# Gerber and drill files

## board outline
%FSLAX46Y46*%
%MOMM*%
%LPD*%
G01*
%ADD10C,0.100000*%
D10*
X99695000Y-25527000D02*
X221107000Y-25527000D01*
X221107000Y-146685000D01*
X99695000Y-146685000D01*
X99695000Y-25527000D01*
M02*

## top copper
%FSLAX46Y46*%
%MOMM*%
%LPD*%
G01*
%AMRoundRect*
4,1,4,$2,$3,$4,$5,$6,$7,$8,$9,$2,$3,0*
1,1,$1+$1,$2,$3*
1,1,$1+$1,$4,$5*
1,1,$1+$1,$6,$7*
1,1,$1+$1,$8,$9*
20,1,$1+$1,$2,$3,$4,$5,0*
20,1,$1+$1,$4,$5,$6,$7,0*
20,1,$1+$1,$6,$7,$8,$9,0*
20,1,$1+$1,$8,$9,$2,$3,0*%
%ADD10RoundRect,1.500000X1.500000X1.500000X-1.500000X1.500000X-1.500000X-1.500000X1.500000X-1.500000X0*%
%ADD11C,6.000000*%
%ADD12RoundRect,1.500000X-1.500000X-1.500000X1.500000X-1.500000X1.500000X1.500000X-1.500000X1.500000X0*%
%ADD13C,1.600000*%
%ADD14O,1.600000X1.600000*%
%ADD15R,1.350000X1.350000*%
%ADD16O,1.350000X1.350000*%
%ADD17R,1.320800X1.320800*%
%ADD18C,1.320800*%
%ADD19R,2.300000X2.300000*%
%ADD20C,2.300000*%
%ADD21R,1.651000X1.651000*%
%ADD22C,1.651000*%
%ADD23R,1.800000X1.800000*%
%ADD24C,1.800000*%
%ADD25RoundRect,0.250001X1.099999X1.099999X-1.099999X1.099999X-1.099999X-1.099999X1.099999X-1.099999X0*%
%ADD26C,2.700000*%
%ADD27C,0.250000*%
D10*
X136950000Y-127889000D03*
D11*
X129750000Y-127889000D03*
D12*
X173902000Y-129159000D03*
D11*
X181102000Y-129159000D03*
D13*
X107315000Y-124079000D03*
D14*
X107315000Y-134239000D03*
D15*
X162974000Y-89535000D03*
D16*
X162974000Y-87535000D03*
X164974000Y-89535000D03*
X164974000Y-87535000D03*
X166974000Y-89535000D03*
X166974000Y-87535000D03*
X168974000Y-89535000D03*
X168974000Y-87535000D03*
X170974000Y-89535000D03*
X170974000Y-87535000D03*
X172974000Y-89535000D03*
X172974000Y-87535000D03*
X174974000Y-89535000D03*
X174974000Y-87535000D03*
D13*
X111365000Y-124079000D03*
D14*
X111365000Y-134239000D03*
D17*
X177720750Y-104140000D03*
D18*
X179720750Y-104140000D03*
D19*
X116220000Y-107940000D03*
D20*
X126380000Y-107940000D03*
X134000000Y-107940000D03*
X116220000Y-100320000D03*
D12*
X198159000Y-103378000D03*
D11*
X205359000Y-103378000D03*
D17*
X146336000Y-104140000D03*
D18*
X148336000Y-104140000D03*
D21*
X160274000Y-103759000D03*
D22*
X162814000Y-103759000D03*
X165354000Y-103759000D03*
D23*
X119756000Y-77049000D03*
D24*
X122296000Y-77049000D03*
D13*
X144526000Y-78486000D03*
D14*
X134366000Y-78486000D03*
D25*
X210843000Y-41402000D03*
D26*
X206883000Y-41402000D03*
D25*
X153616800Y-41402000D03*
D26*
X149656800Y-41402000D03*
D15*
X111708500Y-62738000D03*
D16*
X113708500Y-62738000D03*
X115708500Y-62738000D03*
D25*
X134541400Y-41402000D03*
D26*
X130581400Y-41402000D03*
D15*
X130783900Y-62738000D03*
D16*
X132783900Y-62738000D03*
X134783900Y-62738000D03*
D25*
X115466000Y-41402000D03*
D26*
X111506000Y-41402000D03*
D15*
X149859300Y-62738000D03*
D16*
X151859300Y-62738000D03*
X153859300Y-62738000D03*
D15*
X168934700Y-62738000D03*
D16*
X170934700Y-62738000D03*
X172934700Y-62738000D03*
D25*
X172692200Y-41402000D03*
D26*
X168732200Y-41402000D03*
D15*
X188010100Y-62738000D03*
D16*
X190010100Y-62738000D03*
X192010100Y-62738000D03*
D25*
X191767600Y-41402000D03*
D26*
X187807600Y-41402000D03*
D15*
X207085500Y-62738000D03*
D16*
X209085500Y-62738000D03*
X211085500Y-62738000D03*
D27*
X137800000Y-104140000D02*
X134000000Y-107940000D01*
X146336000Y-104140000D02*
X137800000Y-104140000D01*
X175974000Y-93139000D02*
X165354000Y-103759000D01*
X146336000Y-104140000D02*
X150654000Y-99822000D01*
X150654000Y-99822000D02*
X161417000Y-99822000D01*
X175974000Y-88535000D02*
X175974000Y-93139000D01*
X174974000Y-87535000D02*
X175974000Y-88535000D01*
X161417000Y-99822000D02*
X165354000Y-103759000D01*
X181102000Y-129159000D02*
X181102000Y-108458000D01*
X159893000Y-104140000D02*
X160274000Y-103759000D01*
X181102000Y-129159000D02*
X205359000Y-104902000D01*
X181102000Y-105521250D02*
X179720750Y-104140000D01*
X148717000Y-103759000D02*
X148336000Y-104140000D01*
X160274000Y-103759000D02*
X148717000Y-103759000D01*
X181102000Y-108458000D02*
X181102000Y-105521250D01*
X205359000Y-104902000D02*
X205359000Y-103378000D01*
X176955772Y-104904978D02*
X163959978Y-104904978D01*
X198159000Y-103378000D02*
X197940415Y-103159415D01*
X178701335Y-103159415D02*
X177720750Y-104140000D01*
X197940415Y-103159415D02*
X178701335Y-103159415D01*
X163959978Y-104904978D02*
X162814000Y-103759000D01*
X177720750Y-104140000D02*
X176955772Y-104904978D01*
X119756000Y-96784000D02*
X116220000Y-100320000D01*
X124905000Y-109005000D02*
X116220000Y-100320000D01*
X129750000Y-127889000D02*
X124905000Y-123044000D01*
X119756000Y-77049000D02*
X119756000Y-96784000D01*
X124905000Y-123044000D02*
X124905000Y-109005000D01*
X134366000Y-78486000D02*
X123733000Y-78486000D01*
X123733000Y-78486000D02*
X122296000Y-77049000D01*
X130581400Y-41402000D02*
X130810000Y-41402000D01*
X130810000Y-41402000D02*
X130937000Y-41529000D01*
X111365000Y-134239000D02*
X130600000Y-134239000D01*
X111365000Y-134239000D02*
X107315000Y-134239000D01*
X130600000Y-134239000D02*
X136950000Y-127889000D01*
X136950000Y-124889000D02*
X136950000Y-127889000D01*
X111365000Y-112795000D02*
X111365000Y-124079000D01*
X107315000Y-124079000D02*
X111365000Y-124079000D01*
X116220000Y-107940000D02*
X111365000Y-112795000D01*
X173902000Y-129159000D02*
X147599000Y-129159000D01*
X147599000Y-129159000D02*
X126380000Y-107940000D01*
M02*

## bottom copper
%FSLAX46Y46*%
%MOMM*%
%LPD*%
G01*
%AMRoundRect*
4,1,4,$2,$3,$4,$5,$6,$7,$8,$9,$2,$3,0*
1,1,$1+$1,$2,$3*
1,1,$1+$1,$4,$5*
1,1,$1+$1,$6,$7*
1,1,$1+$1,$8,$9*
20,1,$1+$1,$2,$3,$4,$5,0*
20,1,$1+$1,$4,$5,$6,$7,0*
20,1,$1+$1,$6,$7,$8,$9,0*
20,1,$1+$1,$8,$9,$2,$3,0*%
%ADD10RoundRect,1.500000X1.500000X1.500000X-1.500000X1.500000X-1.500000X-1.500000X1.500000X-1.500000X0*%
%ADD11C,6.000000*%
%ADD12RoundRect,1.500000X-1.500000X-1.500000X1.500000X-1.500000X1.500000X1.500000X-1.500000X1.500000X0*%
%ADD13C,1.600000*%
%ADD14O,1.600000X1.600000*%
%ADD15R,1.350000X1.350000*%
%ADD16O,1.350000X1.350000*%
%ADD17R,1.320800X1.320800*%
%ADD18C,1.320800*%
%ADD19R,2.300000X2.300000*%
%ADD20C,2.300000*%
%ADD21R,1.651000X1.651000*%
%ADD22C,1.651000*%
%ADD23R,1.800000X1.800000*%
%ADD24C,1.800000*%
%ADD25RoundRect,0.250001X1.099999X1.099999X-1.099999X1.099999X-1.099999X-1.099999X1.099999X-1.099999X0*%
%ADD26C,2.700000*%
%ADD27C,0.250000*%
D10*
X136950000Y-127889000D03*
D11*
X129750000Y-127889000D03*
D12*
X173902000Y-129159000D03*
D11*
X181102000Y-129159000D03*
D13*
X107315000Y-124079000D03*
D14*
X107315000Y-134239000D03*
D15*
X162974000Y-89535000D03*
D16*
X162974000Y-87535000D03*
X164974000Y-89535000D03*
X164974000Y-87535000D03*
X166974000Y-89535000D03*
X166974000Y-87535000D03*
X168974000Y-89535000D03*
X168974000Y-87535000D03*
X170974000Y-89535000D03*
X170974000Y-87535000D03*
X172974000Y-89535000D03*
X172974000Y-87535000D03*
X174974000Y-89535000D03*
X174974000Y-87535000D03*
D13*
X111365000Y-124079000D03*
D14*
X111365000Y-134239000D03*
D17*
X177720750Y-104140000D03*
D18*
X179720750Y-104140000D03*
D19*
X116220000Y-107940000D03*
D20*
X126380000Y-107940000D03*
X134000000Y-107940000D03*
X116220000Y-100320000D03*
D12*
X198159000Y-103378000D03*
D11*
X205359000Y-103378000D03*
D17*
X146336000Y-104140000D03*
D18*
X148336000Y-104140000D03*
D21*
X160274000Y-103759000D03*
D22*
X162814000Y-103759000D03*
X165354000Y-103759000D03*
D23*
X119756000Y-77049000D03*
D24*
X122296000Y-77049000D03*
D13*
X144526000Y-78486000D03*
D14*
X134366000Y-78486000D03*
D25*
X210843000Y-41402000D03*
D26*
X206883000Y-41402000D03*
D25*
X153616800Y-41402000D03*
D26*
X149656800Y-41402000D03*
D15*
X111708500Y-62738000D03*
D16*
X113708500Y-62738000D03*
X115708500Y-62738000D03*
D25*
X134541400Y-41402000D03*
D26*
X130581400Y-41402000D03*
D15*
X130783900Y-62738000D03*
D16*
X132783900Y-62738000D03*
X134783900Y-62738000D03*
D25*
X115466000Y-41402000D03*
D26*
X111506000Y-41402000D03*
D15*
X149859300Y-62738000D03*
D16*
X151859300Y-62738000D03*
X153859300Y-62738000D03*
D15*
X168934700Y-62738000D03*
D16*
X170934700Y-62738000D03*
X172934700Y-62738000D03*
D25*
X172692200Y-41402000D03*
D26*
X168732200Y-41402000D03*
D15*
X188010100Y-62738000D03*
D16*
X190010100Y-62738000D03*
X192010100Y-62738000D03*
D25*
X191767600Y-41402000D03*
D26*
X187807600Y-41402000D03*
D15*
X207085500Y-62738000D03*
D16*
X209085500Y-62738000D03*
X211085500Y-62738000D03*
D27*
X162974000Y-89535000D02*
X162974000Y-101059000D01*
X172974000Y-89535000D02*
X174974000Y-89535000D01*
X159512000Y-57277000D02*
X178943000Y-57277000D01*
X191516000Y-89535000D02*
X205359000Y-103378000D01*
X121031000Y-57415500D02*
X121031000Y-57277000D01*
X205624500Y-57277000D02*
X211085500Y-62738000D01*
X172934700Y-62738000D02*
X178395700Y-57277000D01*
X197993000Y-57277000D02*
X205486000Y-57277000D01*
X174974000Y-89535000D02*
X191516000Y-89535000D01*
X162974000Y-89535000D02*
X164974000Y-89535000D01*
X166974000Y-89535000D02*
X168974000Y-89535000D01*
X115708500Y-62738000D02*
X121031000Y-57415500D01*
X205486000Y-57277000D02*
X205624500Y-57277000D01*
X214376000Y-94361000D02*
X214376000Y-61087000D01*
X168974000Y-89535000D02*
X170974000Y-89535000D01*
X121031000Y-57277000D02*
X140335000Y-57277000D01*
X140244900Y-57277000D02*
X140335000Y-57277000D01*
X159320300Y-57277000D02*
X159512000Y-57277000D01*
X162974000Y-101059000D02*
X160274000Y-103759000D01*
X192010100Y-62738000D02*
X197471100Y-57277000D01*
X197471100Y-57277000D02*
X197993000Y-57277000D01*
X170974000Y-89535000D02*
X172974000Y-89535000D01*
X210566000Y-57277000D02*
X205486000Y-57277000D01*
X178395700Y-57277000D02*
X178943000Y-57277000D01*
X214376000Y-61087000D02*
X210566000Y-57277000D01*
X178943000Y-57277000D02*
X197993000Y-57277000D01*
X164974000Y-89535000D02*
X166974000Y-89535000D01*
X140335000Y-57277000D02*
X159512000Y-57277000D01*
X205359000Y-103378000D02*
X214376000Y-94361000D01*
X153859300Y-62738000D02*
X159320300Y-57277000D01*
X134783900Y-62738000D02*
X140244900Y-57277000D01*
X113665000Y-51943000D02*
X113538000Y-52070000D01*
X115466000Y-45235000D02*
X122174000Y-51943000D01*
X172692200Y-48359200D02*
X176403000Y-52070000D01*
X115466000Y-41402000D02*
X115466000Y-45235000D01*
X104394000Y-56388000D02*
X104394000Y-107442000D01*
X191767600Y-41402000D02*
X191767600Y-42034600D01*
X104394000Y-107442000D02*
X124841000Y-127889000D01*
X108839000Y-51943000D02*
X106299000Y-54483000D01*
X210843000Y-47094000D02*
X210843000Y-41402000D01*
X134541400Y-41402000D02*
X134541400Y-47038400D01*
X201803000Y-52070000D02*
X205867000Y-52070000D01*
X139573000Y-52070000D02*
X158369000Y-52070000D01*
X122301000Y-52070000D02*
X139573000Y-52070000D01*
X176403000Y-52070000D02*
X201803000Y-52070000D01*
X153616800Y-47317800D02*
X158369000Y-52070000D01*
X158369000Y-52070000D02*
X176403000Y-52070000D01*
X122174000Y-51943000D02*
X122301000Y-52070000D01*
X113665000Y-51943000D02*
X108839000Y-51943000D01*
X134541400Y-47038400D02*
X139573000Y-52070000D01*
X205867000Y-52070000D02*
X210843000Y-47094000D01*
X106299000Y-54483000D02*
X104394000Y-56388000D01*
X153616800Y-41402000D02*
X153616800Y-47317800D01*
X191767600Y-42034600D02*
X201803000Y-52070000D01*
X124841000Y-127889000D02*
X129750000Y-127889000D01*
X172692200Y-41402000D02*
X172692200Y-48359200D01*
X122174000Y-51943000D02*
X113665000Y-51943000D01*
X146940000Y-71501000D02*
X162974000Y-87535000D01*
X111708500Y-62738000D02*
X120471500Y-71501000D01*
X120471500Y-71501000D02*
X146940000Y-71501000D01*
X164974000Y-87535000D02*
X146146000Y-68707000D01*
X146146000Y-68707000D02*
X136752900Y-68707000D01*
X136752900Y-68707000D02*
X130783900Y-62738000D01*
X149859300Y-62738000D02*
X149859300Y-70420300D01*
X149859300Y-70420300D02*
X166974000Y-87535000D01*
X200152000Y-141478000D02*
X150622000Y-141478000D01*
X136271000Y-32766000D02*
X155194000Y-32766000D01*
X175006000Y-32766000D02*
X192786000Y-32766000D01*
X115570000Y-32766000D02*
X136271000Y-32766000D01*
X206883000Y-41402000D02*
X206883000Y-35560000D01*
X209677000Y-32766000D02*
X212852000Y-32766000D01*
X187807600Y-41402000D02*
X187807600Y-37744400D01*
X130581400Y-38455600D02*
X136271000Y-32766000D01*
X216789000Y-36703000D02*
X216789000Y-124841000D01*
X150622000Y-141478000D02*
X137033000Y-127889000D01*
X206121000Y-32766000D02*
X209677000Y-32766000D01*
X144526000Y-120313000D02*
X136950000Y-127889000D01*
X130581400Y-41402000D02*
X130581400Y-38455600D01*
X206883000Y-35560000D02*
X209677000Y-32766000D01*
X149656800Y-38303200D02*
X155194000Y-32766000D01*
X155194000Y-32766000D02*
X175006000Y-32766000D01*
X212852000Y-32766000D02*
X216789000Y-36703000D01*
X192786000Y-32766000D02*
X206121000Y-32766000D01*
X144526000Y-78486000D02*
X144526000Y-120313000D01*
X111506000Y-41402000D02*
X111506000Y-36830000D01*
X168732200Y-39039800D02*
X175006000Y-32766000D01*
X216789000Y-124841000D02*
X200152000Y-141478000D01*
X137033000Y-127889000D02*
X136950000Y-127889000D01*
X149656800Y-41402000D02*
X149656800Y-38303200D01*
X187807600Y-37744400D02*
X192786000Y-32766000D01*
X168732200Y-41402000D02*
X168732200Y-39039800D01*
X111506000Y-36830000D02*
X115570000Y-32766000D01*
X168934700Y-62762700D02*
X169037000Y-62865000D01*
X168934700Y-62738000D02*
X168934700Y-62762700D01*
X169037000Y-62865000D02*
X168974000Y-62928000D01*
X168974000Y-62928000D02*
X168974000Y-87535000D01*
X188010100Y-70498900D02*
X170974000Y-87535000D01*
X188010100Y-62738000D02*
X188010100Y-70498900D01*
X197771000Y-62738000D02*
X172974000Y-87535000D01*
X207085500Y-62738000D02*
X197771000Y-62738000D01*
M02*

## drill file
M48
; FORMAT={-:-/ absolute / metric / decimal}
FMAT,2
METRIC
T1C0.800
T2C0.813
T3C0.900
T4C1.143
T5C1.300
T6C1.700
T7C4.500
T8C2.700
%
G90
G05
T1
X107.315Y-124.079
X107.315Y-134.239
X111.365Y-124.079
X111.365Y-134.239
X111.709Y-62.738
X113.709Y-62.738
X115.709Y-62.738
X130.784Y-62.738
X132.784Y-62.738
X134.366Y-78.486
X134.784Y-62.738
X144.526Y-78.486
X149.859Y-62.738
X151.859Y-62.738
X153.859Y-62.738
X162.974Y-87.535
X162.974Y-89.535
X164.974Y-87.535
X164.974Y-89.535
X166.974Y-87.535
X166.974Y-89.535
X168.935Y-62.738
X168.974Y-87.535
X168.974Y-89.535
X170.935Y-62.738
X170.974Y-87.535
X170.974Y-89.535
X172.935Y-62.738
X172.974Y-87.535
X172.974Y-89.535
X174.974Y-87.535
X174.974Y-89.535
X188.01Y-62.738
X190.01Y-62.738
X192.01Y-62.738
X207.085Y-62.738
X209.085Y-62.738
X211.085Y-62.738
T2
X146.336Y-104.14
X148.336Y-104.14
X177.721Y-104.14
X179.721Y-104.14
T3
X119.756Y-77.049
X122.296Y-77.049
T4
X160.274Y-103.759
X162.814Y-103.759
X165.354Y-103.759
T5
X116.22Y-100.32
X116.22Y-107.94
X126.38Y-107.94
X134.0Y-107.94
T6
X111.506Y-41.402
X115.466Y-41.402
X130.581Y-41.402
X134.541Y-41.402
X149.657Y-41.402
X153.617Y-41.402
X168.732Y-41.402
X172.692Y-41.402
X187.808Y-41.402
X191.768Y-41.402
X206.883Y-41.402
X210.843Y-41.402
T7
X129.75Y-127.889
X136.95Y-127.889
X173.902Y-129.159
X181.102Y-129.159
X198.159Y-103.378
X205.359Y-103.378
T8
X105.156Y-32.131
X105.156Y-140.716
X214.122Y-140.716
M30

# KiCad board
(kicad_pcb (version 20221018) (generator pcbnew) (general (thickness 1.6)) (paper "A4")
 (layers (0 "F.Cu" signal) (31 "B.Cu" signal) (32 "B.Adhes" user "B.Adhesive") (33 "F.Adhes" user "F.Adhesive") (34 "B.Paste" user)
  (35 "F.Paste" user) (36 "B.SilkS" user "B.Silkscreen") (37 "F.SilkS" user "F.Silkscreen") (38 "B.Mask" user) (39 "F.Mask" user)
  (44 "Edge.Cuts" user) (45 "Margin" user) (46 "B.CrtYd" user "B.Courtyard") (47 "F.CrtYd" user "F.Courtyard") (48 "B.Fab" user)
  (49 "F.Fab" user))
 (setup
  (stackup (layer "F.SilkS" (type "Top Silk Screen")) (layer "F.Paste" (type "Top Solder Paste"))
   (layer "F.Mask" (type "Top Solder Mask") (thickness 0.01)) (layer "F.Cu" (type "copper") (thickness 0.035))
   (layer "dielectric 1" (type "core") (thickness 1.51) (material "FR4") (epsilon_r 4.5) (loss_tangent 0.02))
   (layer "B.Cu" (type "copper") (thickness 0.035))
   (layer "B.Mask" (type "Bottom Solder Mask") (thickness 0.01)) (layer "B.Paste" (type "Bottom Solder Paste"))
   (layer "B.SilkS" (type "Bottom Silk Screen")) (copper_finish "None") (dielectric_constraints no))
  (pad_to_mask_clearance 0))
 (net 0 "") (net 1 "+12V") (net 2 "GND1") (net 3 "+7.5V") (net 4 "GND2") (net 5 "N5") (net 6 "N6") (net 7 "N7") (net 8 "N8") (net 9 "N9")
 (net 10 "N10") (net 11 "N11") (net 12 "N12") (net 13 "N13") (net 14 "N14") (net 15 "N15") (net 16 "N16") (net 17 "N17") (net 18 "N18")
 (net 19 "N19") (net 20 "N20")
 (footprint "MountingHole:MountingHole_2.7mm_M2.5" (layer "F.Cu") (at 214.122 140.716)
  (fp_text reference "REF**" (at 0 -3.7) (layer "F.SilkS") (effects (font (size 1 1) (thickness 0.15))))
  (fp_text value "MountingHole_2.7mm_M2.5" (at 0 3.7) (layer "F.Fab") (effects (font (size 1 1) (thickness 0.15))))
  (pad "" np_thru_hole circle (at 0 0) (size 2.7 2.7) (drill 2.7) (layers "F&B.Cu" "*.Mask")))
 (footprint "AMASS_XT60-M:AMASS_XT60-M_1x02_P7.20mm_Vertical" (layer "F.Cu") (at 136.95 127.889 180)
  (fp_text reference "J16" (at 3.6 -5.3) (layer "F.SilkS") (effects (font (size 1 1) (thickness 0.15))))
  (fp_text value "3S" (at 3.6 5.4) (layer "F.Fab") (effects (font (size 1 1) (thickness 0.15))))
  (pad "1" thru_hole roundrect (at 0 0 180) (size 6 6) (drill 4.5) (layers "*.Cu" "*.Mask") (roundrect_rratio 0.25) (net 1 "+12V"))
  (pad "2" thru_hole circle (at 7.2 0 180) (size 6 6) (drill 4.5) (layers "*.Cu" "*.Mask") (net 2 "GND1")))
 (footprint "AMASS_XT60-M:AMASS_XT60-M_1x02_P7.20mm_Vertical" (layer "F.Cu") (at 173.902 129.159)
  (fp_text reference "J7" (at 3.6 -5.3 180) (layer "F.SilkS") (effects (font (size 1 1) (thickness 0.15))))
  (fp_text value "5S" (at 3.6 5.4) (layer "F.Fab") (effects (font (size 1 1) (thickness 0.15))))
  (pad "1" thru_hole roundrect (at 0 0) (size 6 6) (drill 4.5) (layers "*.Cu" "*.Mask") (roundrect_rratio 0.25) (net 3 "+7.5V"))
  (pad "2" thru_hole circle (at 7.2 0) (size 6 6) (drill 4.5) (layers "*.Cu" "*.Mask") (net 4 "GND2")))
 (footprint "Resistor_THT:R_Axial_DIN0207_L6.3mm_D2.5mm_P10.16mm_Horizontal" (layer "F.Cu") (at 107.315 124.079 -90)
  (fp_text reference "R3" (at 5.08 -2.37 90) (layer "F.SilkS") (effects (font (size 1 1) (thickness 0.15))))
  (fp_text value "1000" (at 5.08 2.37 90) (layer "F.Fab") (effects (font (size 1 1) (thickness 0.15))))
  (pad "1" thru_hole circle (at 0 0 270) (size 1.6 1.6) (drill 0.8) (layers "*.Cu" "*.Mask") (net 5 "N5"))
  (pad "2" thru_hole oval (at 10.16 0 270) (size 1.6 1.6) (drill 0.8) (layers "*.Cu" "*.Mask") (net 1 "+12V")))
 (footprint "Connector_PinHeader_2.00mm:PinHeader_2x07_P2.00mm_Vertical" (layer "F.Cu") (at 162.974 89.535 90)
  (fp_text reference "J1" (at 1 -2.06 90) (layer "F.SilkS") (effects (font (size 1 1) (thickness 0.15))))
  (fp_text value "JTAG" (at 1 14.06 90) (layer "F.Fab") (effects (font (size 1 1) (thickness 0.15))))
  (pad "1" thru_hole rect (at 0 0 90) (size 1.35 1.35) (drill 0.8) (layers "*.Cu" "*.Mask") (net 4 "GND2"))
  (pad "2" thru_hole oval (at 2 0 90) (size 1.35 1.35) (drill 0.8) (layers "*.Cu" "*.Mask") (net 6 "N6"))
  (pad "3" thru_hole oval (at 0 2 90) (size 1.35 1.35) (drill 0.8) (layers "*.Cu" "*.Mask") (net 4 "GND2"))
  (pad "4" thru_hole oval (at 2 2 90) (size 1.35 1.35) (drill 0.8) (layers "*.Cu" "*.Mask") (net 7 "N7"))
  (pad "5" thru_hole oval (at 0 4 90) (size 1.35 1.35) (drill 0.8) (layers "*.Cu" "*.Mask") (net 4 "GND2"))
  (pad "6" thru_hole oval (at 2 4 90) (size 1.35 1.35) (drill 0.8) (layers "*.Cu" "*.Mask") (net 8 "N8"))
  (pad "7" thru_hole oval (at 0 6 90) (size 1.35 1.35) (drill 0.8) (layers "*.Cu" "*.Mask") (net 4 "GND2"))
  (pad "8" thru_hole oval (at 2 6 90) (size 1.35 1.35) (drill 0.8) (layers "*.Cu" "*.Mask") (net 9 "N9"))
  (pad "9" thru_hole oval (at 0 8 90) (size 1.35 1.35) (drill 0.8) (layers "*.Cu" "*.Mask") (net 4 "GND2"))
  (pad "10" thru_hole oval (at 2 8 90) (size 1.35 1.35) (drill 0.8) (layers "*.Cu" "*.Mask") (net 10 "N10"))
  (pad "11" thru_hole oval (at 0 10 90) (size 1.35 1.35) (drill 0.8) (layers "*.Cu" "*.Mask") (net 4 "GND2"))
  (pad "12" thru_hole oval (at 2 10 90) (size 1.35 1.35) (drill 0.8) (layers "*.Cu" "*.Mask") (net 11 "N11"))
  (pad "13" thru_hole oval (at 0 12 90) (size 1.35 1.35) (drill 0.8) (layers "*.Cu" "*.Mask") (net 4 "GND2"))
  (pad "14" thru_hole oval (at 2 12 90) (size 1.35 1.35) (drill 0.8) (layers "*.Cu" "*.Mask") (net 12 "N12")))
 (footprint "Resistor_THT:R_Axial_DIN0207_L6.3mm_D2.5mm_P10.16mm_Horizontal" (layer "F.Cu") (at 111.365 124.079 -90)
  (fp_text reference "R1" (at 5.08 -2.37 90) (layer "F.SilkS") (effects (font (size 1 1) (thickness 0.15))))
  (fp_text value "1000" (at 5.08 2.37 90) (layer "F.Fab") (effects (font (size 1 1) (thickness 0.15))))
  (pad "1" thru_hole circle (at 0 0 270) (size 1.6 1.6) (drill 0.8) (layers "*.Cu" "*.Mask") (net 5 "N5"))
  (pad "2" thru_hole oval (at 10.16 0 270) (size 1.6 1.6) (drill 0.8) (layers "*.Cu" "*.Mask") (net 1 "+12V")))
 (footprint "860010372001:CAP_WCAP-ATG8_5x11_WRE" (layer "F.Cu") (at 177.72075 104.14)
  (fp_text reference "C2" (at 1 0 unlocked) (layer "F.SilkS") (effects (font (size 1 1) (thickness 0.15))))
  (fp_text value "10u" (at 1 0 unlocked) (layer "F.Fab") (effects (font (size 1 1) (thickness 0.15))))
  (pad "1" thru_hole rect (at 0 0) (size 1.3208 1.3208) (drill 0.8128) (layers "*.Cu" "*.Mask") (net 12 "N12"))
  (pad "2" thru_hole circle (at 2 0) (size 1.3208 1.3208) (drill 0.8128) (layers "*.Cu" "*.Mask") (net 4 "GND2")))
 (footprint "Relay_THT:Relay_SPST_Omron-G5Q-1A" (layer "F.Cu") (at 116.22 107.94)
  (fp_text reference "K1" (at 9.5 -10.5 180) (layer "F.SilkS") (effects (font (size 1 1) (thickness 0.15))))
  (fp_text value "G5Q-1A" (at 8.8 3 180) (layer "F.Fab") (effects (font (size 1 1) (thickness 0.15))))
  (pad "1" thru_hole rect (at 0 0 180) (size 2.3 2.3) (drill 1.3) (layers "*.Cu" "*.Mask") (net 5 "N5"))
  (pad "2" thru_hole circle (at 10.16 0 180) (size 2.3 2.3) (drill 1.3) (layers "*.Cu" "*.Mask") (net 3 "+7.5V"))
  (pad "3" thru_hole circle (at 17.78 0 180) (size 2.3 2.3) (drill 1.3) (layers "*.Cu" "*.Mask") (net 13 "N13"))
  (pad "5" thru_hole circle (at 0 -7.62 180) (size 2.3 2.3) (drill 1.3) (layers "*.Cu" "*.Mask") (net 2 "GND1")))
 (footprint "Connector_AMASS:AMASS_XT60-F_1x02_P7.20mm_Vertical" (layer "F.Cu") (at 198.159 103.378)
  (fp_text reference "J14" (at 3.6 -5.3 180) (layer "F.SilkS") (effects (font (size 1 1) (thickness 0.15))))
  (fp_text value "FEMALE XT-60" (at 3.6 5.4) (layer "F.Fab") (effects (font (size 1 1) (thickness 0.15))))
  (pad "1" thru_hole roundrect (at 0 0) (size 6 6) (drill 4.5) (layers "*.Cu" "*.Mask") (roundrect_rratio 0.25) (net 12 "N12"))
  (pad "2" thru_hole circle (at 7.2 0) (size 6 6) (drill 4.5) (layers "*.Cu" "*.Mask") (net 4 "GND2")))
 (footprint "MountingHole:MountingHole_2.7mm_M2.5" (layer "F.Cu") (at 105.156 140.716)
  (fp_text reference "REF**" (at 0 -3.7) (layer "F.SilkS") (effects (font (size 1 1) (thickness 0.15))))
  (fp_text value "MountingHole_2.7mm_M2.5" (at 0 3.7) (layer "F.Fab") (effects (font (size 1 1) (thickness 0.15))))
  (pad "" np_thru_hole circle (at 0 0) (size 2.7 2.7) (drill 2.7) (layers "F&B.Cu" "*.Mask")))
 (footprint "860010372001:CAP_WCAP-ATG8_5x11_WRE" (layer "F.Cu") (at 146.336 104.14)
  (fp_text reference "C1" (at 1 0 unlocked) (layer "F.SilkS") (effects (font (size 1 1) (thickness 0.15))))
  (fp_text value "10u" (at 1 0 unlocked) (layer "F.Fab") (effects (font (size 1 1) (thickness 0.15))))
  (pad "1" thru_hole rect (at 0 0) (size 1.3208 1.3208) (drill 0.8128) (layers "*.Cu" "*.Mask") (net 13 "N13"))
  (pad "2" thru_hole circle (at 2 0) (size 1.3208 1.3208) (drill 0.8128) (layers "*.Cu" "*.Mask") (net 4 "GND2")))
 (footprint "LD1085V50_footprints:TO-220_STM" (layer "F.Cu") (at 160.274 103.759)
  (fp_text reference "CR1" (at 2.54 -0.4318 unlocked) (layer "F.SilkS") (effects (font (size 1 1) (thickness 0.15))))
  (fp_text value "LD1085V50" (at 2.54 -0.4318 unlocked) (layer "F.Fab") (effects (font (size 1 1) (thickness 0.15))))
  (pad "1" thru_hole rect (at 0 0) (size 1.651 1.651) (drill 1.143) (layers "*.Cu" "*.Mask") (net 4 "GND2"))
  (pad "2" thru_hole circle (at 2.54 0) (size 1.651 1.651) (drill 1.143) (layers "*.Cu" "*.Mask") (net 12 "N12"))
  (pad "3" thru_hole circle (at 5.08 0) (size 1.651 1.651) (drill 1.143) (layers "*.Cu" "*.Mask") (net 13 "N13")))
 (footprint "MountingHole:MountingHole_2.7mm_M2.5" (layer "F.Cu") (at 105.156 32.131)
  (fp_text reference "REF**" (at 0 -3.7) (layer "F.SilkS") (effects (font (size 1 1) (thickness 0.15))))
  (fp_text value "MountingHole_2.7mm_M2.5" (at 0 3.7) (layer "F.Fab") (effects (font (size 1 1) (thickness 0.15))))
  (pad "" np_thru_hole circle (at 0 0) (size 2.7 2.7) (drill 2.7) (layers "*.Cu" "*.Mask")))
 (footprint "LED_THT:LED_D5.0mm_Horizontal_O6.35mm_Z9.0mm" (layer "F.Cu") (at 119.756 77.049)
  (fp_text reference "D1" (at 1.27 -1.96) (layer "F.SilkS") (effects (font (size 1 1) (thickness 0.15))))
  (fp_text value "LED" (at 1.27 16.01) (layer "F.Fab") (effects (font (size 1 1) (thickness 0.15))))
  (pad "1" thru_hole rect (at 0 0) (size 1.8 1.8) (drill 0.9) (layers "*.Cu" "*.Mask") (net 2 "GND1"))
  (pad "2" thru_hole circle (at 2.54 0) (size 1.8 1.8) (drill 0.9) (layers "*.Cu" "*.Mask") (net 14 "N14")))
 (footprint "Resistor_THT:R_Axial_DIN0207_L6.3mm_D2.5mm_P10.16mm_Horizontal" (layer "F.Cu") (at 144.526 78.486 180)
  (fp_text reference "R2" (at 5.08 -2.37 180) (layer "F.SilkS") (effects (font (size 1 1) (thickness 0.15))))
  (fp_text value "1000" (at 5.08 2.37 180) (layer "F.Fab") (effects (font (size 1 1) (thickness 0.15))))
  (pad "1" thru_hole circle (at 0 0 180) (size 1.6 1.6) (drill 0.8) (layers "*.Cu" "*.Mask") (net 1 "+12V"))
  (pad "2" thru_hole oval (at 10.16 0 180) (size 1.6 1.6) (drill 0.8) (layers "*.Cu" "*.Mask") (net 14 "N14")))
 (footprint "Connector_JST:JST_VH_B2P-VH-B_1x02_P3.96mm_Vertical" (layer "B.Cu") (at 210.843 41.402 180)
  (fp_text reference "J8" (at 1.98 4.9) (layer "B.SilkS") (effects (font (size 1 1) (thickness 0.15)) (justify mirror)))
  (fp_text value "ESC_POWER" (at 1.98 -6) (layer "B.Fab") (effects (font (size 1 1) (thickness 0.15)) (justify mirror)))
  (pad "1" thru_hole roundrect (at 0 0 180) (size 2.7 2.7) (drill 1.7) (layers "*.Cu" "*.Mask") (roundrect_rratio 0.09259296296)
   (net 2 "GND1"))
  (pad "2" thru_hole circle (at 3.96 0 180) (size 2.7 2.7) (drill 1.7) (layers "*.Cu" "*.Mask") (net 1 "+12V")))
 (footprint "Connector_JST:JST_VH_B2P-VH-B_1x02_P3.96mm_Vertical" (layer "B.Cu") (at 153.6168 41.402 180)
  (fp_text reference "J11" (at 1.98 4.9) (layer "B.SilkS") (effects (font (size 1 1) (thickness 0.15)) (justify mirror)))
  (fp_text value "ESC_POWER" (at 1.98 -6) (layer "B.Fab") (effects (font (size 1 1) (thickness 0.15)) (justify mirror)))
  (pad "1" thru_hole roundrect (at 0 0 180) (size 2.7 2.7) (drill 1.7) (layers "*.Cu" "*.Mask") (roundrect_rratio 0.09259296296)
   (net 2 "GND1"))
  (pad "2" thru_hole circle (at 3.96 0 180) (size 2.7 2.7) (drill 1.7) (layers "*.Cu" "*.Mask") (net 1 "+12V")))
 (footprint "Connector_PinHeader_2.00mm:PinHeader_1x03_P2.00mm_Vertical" (layer "B.Cu") (at 111.7085 62.738 -90)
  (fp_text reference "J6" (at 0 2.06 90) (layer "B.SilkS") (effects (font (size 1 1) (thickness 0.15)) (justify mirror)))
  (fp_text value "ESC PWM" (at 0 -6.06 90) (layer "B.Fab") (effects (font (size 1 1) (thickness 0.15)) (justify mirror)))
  (pad "1" thru_hole rect (at 0 0 270) (size 1.35 1.35) (drill 0.8) (layers "*.Cu" "*.Mask") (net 6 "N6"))
  (pad "2" thru_hole oval (at 0 -2 270) (size 1.35 1.35) (drill 0.8) (layers "*.Cu" "*.Mask") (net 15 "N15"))
  (pad "3" thru_hole oval (at 0 -4 270) (size 1.35 1.35) (drill 0.8) (layers "*.Cu" "*.Mask") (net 4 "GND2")))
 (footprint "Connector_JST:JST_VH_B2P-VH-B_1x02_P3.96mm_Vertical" (layer "B.Cu") (at 134.5414 41.402 180)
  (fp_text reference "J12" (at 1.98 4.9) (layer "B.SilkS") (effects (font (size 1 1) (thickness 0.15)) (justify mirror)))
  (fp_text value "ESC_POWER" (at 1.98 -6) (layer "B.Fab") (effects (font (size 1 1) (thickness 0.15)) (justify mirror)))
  (pad "1" thru_hole roundrect (at 0 0 180) (size 2.7 2.7) (drill 1.7) (layers "*.Cu" "*.Mask") (roundrect_rratio 0.09259296296)
   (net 2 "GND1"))
  (pad "2" thru_hole circle (at 3.96 0 180) (size 2.7 2.7) (drill 1.7) (layers "*.Cu" "*.Mask") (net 1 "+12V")))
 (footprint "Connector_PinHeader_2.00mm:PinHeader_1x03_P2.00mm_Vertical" (layer "B.Cu") (at 130.7839 62.738 -90)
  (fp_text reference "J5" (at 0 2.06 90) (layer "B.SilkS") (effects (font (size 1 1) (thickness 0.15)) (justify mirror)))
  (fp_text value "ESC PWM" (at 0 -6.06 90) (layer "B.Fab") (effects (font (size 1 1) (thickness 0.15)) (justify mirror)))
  (pad "1" thru_hole rect (at 0 0 270) (size 1.35 1.35) (drill 0.8) (layers "*.Cu" "*.Mask") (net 7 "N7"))
  (pad "2" thru_hole oval (at 0 -2 270) (size 1.35 1.35) (drill 0.8) (layers "*.Cu" "*.Mask") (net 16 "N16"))
  (pad "3" thru_hole oval (at 0 -4 270) (size 1.35 1.35) (drill 0.8) (layers "*.Cu" "*.Mask") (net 4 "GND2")))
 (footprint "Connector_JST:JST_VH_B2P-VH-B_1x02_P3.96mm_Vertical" (layer "B.Cu") (at 115.466 41.402 180)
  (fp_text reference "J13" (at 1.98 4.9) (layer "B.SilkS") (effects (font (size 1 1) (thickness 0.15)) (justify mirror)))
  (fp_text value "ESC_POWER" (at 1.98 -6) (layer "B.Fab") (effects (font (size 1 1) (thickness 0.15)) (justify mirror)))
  (pad "1" thru_hole roundrect (at 0 0 180) (size 2.7 2.7) (drill 1.7) (layers "*.Cu" "*.Mask") (roundrect_rratio 0.09259296296)
   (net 2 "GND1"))
  (pad "2" thru_hole circle (at 3.96 0 180) (size 2.7 2.7) (drill 1.7) (layers "*.Cu" "*.Mask") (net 1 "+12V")))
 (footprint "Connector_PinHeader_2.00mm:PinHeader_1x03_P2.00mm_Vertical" (layer "B.Cu") (at 149.8593 62.738 -90)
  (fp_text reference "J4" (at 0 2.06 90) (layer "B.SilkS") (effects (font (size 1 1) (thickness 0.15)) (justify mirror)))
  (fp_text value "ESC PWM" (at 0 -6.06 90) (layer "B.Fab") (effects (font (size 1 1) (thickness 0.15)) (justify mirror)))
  (pad "1" thru_hole rect (at 0 0 270) (size 1.35 1.35) (drill 0.8) (layers "*.Cu" "*.Mask") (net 8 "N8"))
  (pad "2" thru_hole oval (at 0 -2 270) (size 1.35 1.35) (drill 0.8) (layers "*.Cu" "*.Mask") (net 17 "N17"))
  (pad "3" thru_hole oval (at 0 -4 270) (size 1.35 1.35) (drill 0.8) (layers "*.Cu" "*.Mask") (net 4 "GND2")))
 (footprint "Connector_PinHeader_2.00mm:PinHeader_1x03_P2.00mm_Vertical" (layer "B.Cu") (at 168.9347 62.738 -90)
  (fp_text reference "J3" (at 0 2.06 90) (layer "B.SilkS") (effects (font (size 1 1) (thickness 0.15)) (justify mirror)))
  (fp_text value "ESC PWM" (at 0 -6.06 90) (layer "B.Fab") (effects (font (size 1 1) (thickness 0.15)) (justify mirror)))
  (pad "1" thru_hole rect (at 0 0 270) (size 1.35 1.35) (drill 0.8) (layers "*.Cu" "*.Mask") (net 9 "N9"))
  (pad "2" thru_hole oval (at 0 -2 270) (size 1.35 1.35) (drill 0.8) (layers "*.Cu" "*.Mask") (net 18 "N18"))
  (pad "3" thru_hole oval (at 0 -4 270) (size 1.35 1.35) (drill 0.8) (layers "*.Cu" "*.Mask") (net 4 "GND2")))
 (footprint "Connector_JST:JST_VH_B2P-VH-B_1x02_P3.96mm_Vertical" (layer "B.Cu") (at 172.6922 41.402 180)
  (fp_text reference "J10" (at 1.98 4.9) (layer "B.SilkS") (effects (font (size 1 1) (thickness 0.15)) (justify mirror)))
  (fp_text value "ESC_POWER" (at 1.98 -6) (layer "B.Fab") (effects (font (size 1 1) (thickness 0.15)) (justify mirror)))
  (pad "1" thru_hole roundrect (at 0 0 180) (size 2.7 2.7) (drill 1.7) (layers "*.Cu" "*.Mask") (roundrect_rratio 0.09259296296)
   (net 2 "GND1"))
  (pad "2" thru_hole circle (at 3.96 0 180) (size 2.7 2.7) (drill 1.7) (layers "*.Cu" "*.Mask") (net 1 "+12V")))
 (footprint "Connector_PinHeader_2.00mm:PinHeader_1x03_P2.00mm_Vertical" (layer "B.Cu") (at 188.0101 62.738 -90)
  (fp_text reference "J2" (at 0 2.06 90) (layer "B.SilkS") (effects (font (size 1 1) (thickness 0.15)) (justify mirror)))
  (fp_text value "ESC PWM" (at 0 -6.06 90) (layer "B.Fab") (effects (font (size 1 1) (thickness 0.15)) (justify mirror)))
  (pad "1" thru_hole rect (at 0 0 270) (size 1.35 1.35) (drill 0.8) (layers "*.Cu" "*.Mask") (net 10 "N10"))
  (pad "2" thru_hole oval (at 0 -2 270) (size 1.35 1.35) (drill 0.8) (layers "*.Cu" "*.Mask") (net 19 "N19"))
  (pad "3" thru_hole oval (at 0 -4 270) (size 1.35 1.35) (drill 0.8) (layers "*.Cu" "*.Mask") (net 4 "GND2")))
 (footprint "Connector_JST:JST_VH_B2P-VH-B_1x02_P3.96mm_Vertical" (layer "B.Cu") (at 191.7676 41.402 180)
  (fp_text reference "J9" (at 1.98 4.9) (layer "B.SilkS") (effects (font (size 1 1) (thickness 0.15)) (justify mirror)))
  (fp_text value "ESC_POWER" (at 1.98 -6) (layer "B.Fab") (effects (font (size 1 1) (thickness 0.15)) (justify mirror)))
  (pad "1" thru_hole roundrect (at 0 0 180) (size 2.7 2.7) (drill 1.7) (layers "*.Cu" "*.Mask") (roundrect_rratio 0.09259296296)
   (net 2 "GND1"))
  (pad "2" thru_hole circle (at 3.96 0 180) (size 2.7 2.7) (drill 1.7) (layers "*.Cu" "*.Mask") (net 1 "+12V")))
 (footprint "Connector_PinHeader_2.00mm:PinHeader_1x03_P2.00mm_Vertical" (layer "B.Cu") (at 207.0855 62.738 -90)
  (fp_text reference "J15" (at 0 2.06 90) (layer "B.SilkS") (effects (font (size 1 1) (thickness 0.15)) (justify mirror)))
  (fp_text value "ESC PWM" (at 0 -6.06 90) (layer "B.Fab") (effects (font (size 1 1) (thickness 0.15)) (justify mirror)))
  (pad "1" thru_hole rect (at 0 0 270) (size 1.35 1.35) (drill 0.8) (layers "*.Cu" "*.Mask") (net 11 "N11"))
  (pad "2" thru_hole oval (at 0 -2 270) (size 1.35 1.35) (drill 0.8) (layers "*.Cu" "*.Mask") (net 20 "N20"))
  (pad "3" thru_hole oval (at 0 -4 270) (size 1.35 1.35) (drill 0.8) (layers "*.Cu" "*.Mask") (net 4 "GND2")))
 (gr_rect (start 99.695 25.527) (end 221.107 146.685) (stroke (width 0.1) (type default)) (fill none) (layer "Edge.Cuts"))
 (segment (start 137.8 104.14) (end 134 107.94) (width 0.25) (layer "F.Cu") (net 13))
 (segment (start 146.336 104.14) (end 137.8 104.14) (width 0.25) (layer "F.Cu") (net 13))
 (segment (start 175.974 93.139) (end 165.354 103.759) (width 0.25) (layer "F.Cu") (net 13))
 (segment (start 146.336 104.14) (end 150.654 99.822) (width 0.25) (layer "F.Cu") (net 13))
 (segment (start 150.654 99.822) (end 161.417 99.822) (width 0.25) (layer "F.Cu") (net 13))
 (segment (start 175.974 88.535) (end 175.974 93.139) (width 0.25) (layer "F.Cu") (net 13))
 (segment (start 174.974 87.535) (end 175.974 88.535) (width 0.25) (layer "F.Cu") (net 13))
 (segment (start 161.417 99.822) (end 165.354 103.759) (width 0.25) (layer "F.Cu") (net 13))
 (segment (start 181.102 129.159) (end 181.102 108.458) (width 0.25) (layer "F.Cu") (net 4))
 (segment (start 159.893 104.14) (end 160.274 103.759) (width 0.25) (layer "F.Cu") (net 4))
 (segment (start 181.102 129.159) (end 205.359 104.902) (width 0.25) (layer "F.Cu") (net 4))
 (segment (start 181.102 105.52125) (end 179.72075 104.14) (width 0.25) (layer "F.Cu") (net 4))
 (segment (start 148.717 103.759) (end 148.336 104.14) (width 0.25) (layer "F.Cu") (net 4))
 (segment (start 160.274 103.759) (end 148.717 103.759) (width 0.25) (layer "F.Cu") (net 4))
 (segment (start 181.102 108.458) (end 181.102 105.52125) (width 0.25) (layer "F.Cu") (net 4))
 (segment (start 205.359 104.902) (end 205.359 103.378) (width 0.25) (layer "F.Cu") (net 4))
 (segment (start 162.974 89.535) (end 162.974 101.059) (width 0.25) (layer "B.Cu") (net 4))
 (segment (start 172.974 89.535) (end 174.974 89.535) (width 0.25) (layer "B.Cu") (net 4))
 (segment (start 159.512 57.277) (end 178.943 57.277) (width 0.25) (layer "B.Cu") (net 4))
 (segment (start 191.516 89.535) (end 205.359 103.378) (width 0.25) (layer "B.Cu") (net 4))
 (segment (start 121.031 57.4155) (end 121.031 57.277) (width 0.25) (layer "B.Cu") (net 4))
 (segment (start 205.6245 57.277) (end 211.0855 62.738) (width 0.25) (layer "B.Cu") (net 4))
 (segment (start 172.9347 62.738) (end 178.3957 57.277) (width 0.25) (layer "B.Cu") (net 4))
 (segment (start 197.993 57.277) (end 205.486 57.277) (width 0.25) (layer "B.Cu") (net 4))
 (segment (start 174.974 89.535) (end 191.516 89.535) (width 0.25) (layer "B.Cu") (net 4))
 (segment (start 162.974 89.535) (end 164.974 89.535) (width 0.25) (layer "B.Cu") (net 4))
 (segment (start 166.974 89.535) (end 168.974 89.535) (width 0.25) (layer "B.Cu") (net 4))
 (segment (start 115.7085 62.738) (end 121.031 57.4155) (width 0.25) (layer "B.Cu") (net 4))
 (segment (start 205.486 57.277) (end 205.6245 57.277) (width 0.25) (layer "B.Cu") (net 4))
 (segment (start 214.376 94.361) (end 214.376 61.087) (width 0.25) (layer "B.Cu") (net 4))
 (segment (start 168.974 89.535) (end 170.974 89.535) (width 0.25) (layer "B.Cu") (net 4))
 (segment (start 121.031 57.277) (end 140.335 57.277) (width 0.25) (layer "B.Cu") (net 4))
 (segment (start 140.2449 57.277) (end 140.335 57.277) (width 0.25) (layer "B.Cu") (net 4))
 (segment (start 159.3203 57.277) (end 159.512 57.277) (width 0.25) (layer "B.Cu") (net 4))
 (segment (start 162.974 101.059) (end 160.274 103.759) (width 0.25) (layer "B.Cu") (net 4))
 (segment (start 192.0101 62.738) (end 197.4711 57.277) (width 0.25) (layer "B.Cu") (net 4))
 (segment (start 197.4711 57.277) (end 197.993 57.277) (width 0.25) (layer "B.Cu") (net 4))
 (segment (start 170.974 89.535) (end 172.974 89.535) (width 0.25) (layer "B.Cu") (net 4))
 (segment (start 210.566 57.277) (end 205.486 57.277) (width 0.25) (layer "B.Cu") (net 4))
 (segment (start 178.3957 57.277) (end 178.943 57.277) (width 0.25) (layer "B.Cu") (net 4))
 (segment (start 214.376 61.087) (end 210.566 57.277) (width 0.25) (layer "B.Cu") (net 4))
 (segment (start 178.943 57.277) (end 197.993 57.277) (width 0.25) (layer "B.Cu") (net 4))
 (segment (start 164.974 89.535) (end 166.974 89.535) (width 0.25) (layer "B.Cu") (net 4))
 (segment (start 140.335 57.277) (end 159.512 57.277) (width 0.25) (layer "B.Cu") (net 4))
 (segment (start 205.359 103.378) (end 214.376 94.361) (width 0.25) (layer "B.Cu") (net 4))
 (segment (start 153.8593 62.738) (end 159.3203 57.277) (width 0.25) (layer "B.Cu") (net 4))
 (segment (start 134.7839 62.738) (end 140.2449 57.277) (width 0.25) (layer "B.Cu") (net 4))
 (segment (start 176.955772 104.904978) (end 163.959978 104.904978) (width 0.25) (layer "F.Cu") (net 12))
 (segment (start 198.159 103.378) (end 197.940415 103.159415) (width 0.25) (layer "F.Cu") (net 12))
 (segment (start 178.701335 103.159415) (end 177.72075 104.14) (width 0.25) (layer "F.Cu") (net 12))
 (segment (start 197.940415 103.159415) (end 178.701335 103.159415) (width 0.25) (layer "F.Cu") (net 12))
 (segment (start 163.959978 104.904978) (end 162.814 103.759) (width 0.25) (layer "F.Cu") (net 12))
 (segment (start 177.72075 104.14) (end 176.955772 104.904978) (width 0.25) (layer "F.Cu") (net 12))
 (segment (start 119.756 96.784) (end 116.22 100.32) (width 0.25) (layer "F.Cu") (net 2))
 (segment (start 124.905 109.005) (end 116.22 100.32) (width 0.25) (layer "F.Cu") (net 2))
 (segment (start 129.75 127.889) (end 124.905 123.044) (width 0.25) (layer "F.Cu") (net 2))
 (segment (start 119.756 77.049) (end 119.756 96.784) (width 0.25) (layer "F.Cu") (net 2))
 (segment (start 124.905 123.044) (end 124.905 109.005) (width 0.25) (layer "F.Cu") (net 2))
 (segment (start 113.665 51.943) (end 113.538 52.07) (width 0.25) (layer "B.Cu") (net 2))
 (segment (start 115.466 45.235) (end 122.174 51.943) (width 0.25) (layer "B.Cu") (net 2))
 (segment (start 172.6922 48.3592) (end 176.403 52.07) (width 0.25) (layer "B.Cu") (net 2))
 (segment (start 115.466 41.402) (end 115.466 45.235) (width 0.25) (layer "B.Cu") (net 2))
 (segment (start 104.394 56.388) (end 104.394 107.442) (width 0.25) (layer "B.Cu") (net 2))
 (segment (start 191.7676 41.402) (end 191.7676 42.0346) (width 0.25) (layer "B.Cu") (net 2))
 (segment (start 104.394 107.442) (end 124.841 127.889) (width 0.25) (layer "B.Cu") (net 2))
 (segment (start 108.839 51.943) (end 106.299 54.483) (width 0.25) (layer "B.Cu") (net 2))
 (segment (start 210.843 47.094) (end 210.843 41.402) (width 0.25) (layer "B.Cu") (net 2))
 (segment (start 134.5414 41.402) (end 134.5414 47.0384) (width 0.25) (layer "B.Cu") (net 2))
 (segment (start 201.803 52.07) (end 205.867 52.07) (width 0.25) (layer "B.Cu") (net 2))
 (segment (start 139.573 52.07) (end 158.369 52.07) (width 0.25) (layer "B.Cu") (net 2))
 (segment (start 122.301 52.07) (end 139.573 52.07) (width 0.25) (layer "B.Cu") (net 2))
 (segment (start 176.403 52.07) (end 201.803 52.07) (width 0.25) (layer "B.Cu") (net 2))
 (segment (start 153.6168 47.3178) (end 158.369 52.07) (width 0.25) (layer "B.Cu") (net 2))
 (segment (start 158.369 52.07) (end 176.403 52.07) (width 0.25) (layer "B.Cu") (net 2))
 (segment (start 122.174 51.943) (end 122.301 52.07) (width 0.25) (layer "B.Cu") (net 2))
 (segment (start 113.665 51.943) (end 108.839 51.943) (width 0.25) (layer "B.Cu") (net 2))
 (segment (start 134.5414 47.0384) (end 139.573 52.07) (width 0.25) (layer "B.Cu") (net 2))
 (segment (start 205.867 52.07) (end 210.843 47.094) (width 0.25) (layer "B.Cu") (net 2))
 (segment (start 106.299 54.483) (end 104.394 56.388) (width 0.25) (layer "B.Cu") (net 2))
 (segment (start 153.6168 41.402) (end 153.6168 47.3178) (width 0.25) (layer "B.Cu") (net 2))
 (segment (start 191.7676 42.0346) (end 201.803 52.07) (width 0.25) (layer "B.Cu") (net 2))
 (segment (start 124.841 127.889) (end 129.75 127.889) (width 0.25) (layer "B.Cu") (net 2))
 (segment (start 172.6922 41.402) (end 172.6922 48.3592) (width 0.25) (layer "B.Cu") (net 2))
 (segment (start 122.174 51.943) (end 113.665 51.943) (width 0.25) (layer "B.Cu") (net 2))
 (segment (start 134.366 78.486) (end 123.733 78.486) (width 0.25) (layer "F.Cu") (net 14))
 (segment (start 123.733 78.486) (end 122.296 77.049) (width 0.25) (layer "F.Cu") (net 14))
 (segment (start 146.94 71.501) (end 162.974 87.535) (width 0.25) (layer "B.Cu") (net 6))
 (segment (start 111.7085 62.738) (end 120.4715 71.501) (width 0.25) (layer "B.Cu") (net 6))
 (segment (start 120.4715 71.501) (end 146.94 71.501) (width 0.25) (layer "B.Cu") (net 6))
 (segment (start 164.974 87.535) (end 146.146 68.707) (width 0.25) (layer "B.Cu") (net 7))
 (segment (start 146.146 68.707) (end 136.7529 68.707) (width 0.25) (layer "B.Cu") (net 7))
 (segment (start 136.7529 68.707) (end 130.7839 62.738) (width 0.25) (layer "B.Cu") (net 7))
 (segment (start 149.8593 62.738) (end 149.8593 70.4203) (width 0.25) (layer "B.Cu") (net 8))
 (segment (start 149.8593 70.4203) (end 166.974 87.535) (width 0.25) (layer "B.Cu") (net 8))
 (segment (start 130.5814 41.402) (end 130.81 41.402) (width 0.25) (layer "F.Cu") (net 1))
 (segment (start 130.81 41.402) (end 130.937 41.529) (width 0.25) (layer "F.Cu") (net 1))
 (segment (start 111.365 134.239) (end 130.6 134.239) (width 0.25) (layer "F.Cu") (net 1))
 (segment (start 111.365 134.239) (end 107.315 134.239) (width 0.25) (layer "F.Cu") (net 1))
 (segment (start 130.6 134.239) (end 136.95 127.889) (width 0.25) (layer "F.Cu") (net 1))
 (segment (start 136.95 124.889) (end 136.95 127.889) (width 0.25) (layer "F.Cu") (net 1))
 (segment (start 200.152 141.478) (end 150.622 141.478) (width 0.25) (layer "B.Cu") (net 1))
 (segment (start 136.271 32.766) (end 155.194 32.766) (width 0.25) (layer "B.Cu") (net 1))
 (segment (start 175.006 32.766) (end 192.786 32.766) (width 0.25) (layer "B.Cu") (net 1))
 (segment (start 115.57 32.766) (end 136.271 32.766) (width 0.25) (layer "B.Cu") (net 1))
 (segment (start 206.883 41.402) (end 206.883 35.56) (width 0.25) (layer "B.Cu") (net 1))
 (segment (start 209.677 32.766) (end 212.852 32.766) (width 0.25) (layer "B.Cu") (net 1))
 (segment (start 187.8076 41.402) (end 187.8076 37.7444) (width 0.25) (layer "B.Cu") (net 1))
 (segment (start 130.5814 38.4556) (end 136.271 32.766) (width 0.25) (layer "B.Cu") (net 1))
 (segment (start 216.789 36.703) (end 216.789 124.841) (width 0.25) (layer "B.Cu") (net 1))
 (segment (start 150.622 141.478) (end 137.033 127.889) (width 0.25) (layer "B.Cu") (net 1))
 (segment (start 206.121 32.766) (end 209.677 32.766) (width 0.25) (layer "B.Cu") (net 1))
 (segment (start 144.526 120.313) (end 136.95 127.889) (width 0.25) (layer "B.Cu") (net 1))
 (segment (start 130.5814 41.402) (end 130.5814 38.4556) (width 0.25) (layer "B.Cu") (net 1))
 (segment (start 206.883 35.56) (end 209.677 32.766) (width 0.25) (layer "B.Cu") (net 1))
 (segment (start 149.6568 38.3032) (end 155.194 32.766) (width 0.25) (layer "B.Cu") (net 1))
 (segment (start 155.194 32.766) (end 175.006 32.766) (width 0.25) (layer "B.Cu") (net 1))
 (segment (start 212.852 32.766) (end 216.789 36.703) (width 0.25) (layer "B.Cu") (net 1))
 (segment (start 192.786 32.766) (end 206.121 32.766) (width 0.25) (layer "B.Cu") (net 1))
 (segment (start 144.526 78.486) (end 144.526 120.313) (width 0.25) (layer "B.Cu") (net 1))
 (segment (start 111.506 41.402) (end 111.506 36.83) (width 0.25) (layer "B.Cu") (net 1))
 (segment (start 168.7322 39.0398) (end 175.006 32.766) (width 0.25) (layer "B.Cu") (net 1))
 (segment (start 216.789 124.841) (end 200.152 141.478) (width 0.25) (layer "B.Cu") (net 1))
 (segment (start 137.033 127.889) (end 136.95 127.889) (width 0.25) (layer "B.Cu") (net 1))
 (segment (start 149.6568 41.402) (end 149.6568 38.3032) (width 0.25) (layer "B.Cu") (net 1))
 (segment (start 187.8076 37.7444) (end 192.786 32.766) (width 0.25) (layer "B.Cu") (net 1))
 (segment (start 168.7322 41.402) (end 168.7322 39.0398) (width 0.25) (layer "B.Cu") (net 1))
 (segment (start 111.506 36.83) (end 115.57 32.766) (width 0.25) (layer "B.Cu") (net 1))
 (segment (start 111.365 112.795) (end 111.365 124.079) (width 0.25) (layer "F.Cu") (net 5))
 (segment (start 107.315 124.079) (end 111.365 124.079) (width 0.25) (layer "F.Cu") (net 5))
 (segment (start 116.22 107.94) (end 111.365 112.795) (width 0.25) (layer "F.Cu") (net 5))
 (segment (start 173.902 129.159) (end 147.599 129.159) (width 0.25) (layer "F.Cu") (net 3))
 (segment (start 147.599 129.159) (end 126.38 107.94) (width 0.25) (layer "F.Cu") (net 3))
 (segment (start 168.9347 62.7627) (end 169.037 62.865) (width 0.25) (layer "B.Cu") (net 9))
 (segment (start 168.9347 62.738) (end 168.9347 62.7627) (width 0.25) (layer "B.Cu") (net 9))
 (segment (start 169.037 62.865) (end 168.974 62.928) (width 0.25) (layer "B.Cu") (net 9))
 (segment (start 168.974 62.928) (end 168.974 87.535) (width 0.25) (layer "B.Cu") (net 9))
 (segment (start 188.0101 70.4989) (end 170.974 87.535) (width 0.25) (layer "B.Cu") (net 10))
 (segment (start 188.0101 62.738) (end 188.0101 70.4989) (width 0.25) (layer "B.Cu") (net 10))
 (segment (start 197.771 62.738) (end 172.974 87.535) (width 0.25) (layer "B.Cu") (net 11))
 (segment (start 207.0855 62.738) (end 197.771 62.738) (width 0.25) (layer "B.Cu") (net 11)))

